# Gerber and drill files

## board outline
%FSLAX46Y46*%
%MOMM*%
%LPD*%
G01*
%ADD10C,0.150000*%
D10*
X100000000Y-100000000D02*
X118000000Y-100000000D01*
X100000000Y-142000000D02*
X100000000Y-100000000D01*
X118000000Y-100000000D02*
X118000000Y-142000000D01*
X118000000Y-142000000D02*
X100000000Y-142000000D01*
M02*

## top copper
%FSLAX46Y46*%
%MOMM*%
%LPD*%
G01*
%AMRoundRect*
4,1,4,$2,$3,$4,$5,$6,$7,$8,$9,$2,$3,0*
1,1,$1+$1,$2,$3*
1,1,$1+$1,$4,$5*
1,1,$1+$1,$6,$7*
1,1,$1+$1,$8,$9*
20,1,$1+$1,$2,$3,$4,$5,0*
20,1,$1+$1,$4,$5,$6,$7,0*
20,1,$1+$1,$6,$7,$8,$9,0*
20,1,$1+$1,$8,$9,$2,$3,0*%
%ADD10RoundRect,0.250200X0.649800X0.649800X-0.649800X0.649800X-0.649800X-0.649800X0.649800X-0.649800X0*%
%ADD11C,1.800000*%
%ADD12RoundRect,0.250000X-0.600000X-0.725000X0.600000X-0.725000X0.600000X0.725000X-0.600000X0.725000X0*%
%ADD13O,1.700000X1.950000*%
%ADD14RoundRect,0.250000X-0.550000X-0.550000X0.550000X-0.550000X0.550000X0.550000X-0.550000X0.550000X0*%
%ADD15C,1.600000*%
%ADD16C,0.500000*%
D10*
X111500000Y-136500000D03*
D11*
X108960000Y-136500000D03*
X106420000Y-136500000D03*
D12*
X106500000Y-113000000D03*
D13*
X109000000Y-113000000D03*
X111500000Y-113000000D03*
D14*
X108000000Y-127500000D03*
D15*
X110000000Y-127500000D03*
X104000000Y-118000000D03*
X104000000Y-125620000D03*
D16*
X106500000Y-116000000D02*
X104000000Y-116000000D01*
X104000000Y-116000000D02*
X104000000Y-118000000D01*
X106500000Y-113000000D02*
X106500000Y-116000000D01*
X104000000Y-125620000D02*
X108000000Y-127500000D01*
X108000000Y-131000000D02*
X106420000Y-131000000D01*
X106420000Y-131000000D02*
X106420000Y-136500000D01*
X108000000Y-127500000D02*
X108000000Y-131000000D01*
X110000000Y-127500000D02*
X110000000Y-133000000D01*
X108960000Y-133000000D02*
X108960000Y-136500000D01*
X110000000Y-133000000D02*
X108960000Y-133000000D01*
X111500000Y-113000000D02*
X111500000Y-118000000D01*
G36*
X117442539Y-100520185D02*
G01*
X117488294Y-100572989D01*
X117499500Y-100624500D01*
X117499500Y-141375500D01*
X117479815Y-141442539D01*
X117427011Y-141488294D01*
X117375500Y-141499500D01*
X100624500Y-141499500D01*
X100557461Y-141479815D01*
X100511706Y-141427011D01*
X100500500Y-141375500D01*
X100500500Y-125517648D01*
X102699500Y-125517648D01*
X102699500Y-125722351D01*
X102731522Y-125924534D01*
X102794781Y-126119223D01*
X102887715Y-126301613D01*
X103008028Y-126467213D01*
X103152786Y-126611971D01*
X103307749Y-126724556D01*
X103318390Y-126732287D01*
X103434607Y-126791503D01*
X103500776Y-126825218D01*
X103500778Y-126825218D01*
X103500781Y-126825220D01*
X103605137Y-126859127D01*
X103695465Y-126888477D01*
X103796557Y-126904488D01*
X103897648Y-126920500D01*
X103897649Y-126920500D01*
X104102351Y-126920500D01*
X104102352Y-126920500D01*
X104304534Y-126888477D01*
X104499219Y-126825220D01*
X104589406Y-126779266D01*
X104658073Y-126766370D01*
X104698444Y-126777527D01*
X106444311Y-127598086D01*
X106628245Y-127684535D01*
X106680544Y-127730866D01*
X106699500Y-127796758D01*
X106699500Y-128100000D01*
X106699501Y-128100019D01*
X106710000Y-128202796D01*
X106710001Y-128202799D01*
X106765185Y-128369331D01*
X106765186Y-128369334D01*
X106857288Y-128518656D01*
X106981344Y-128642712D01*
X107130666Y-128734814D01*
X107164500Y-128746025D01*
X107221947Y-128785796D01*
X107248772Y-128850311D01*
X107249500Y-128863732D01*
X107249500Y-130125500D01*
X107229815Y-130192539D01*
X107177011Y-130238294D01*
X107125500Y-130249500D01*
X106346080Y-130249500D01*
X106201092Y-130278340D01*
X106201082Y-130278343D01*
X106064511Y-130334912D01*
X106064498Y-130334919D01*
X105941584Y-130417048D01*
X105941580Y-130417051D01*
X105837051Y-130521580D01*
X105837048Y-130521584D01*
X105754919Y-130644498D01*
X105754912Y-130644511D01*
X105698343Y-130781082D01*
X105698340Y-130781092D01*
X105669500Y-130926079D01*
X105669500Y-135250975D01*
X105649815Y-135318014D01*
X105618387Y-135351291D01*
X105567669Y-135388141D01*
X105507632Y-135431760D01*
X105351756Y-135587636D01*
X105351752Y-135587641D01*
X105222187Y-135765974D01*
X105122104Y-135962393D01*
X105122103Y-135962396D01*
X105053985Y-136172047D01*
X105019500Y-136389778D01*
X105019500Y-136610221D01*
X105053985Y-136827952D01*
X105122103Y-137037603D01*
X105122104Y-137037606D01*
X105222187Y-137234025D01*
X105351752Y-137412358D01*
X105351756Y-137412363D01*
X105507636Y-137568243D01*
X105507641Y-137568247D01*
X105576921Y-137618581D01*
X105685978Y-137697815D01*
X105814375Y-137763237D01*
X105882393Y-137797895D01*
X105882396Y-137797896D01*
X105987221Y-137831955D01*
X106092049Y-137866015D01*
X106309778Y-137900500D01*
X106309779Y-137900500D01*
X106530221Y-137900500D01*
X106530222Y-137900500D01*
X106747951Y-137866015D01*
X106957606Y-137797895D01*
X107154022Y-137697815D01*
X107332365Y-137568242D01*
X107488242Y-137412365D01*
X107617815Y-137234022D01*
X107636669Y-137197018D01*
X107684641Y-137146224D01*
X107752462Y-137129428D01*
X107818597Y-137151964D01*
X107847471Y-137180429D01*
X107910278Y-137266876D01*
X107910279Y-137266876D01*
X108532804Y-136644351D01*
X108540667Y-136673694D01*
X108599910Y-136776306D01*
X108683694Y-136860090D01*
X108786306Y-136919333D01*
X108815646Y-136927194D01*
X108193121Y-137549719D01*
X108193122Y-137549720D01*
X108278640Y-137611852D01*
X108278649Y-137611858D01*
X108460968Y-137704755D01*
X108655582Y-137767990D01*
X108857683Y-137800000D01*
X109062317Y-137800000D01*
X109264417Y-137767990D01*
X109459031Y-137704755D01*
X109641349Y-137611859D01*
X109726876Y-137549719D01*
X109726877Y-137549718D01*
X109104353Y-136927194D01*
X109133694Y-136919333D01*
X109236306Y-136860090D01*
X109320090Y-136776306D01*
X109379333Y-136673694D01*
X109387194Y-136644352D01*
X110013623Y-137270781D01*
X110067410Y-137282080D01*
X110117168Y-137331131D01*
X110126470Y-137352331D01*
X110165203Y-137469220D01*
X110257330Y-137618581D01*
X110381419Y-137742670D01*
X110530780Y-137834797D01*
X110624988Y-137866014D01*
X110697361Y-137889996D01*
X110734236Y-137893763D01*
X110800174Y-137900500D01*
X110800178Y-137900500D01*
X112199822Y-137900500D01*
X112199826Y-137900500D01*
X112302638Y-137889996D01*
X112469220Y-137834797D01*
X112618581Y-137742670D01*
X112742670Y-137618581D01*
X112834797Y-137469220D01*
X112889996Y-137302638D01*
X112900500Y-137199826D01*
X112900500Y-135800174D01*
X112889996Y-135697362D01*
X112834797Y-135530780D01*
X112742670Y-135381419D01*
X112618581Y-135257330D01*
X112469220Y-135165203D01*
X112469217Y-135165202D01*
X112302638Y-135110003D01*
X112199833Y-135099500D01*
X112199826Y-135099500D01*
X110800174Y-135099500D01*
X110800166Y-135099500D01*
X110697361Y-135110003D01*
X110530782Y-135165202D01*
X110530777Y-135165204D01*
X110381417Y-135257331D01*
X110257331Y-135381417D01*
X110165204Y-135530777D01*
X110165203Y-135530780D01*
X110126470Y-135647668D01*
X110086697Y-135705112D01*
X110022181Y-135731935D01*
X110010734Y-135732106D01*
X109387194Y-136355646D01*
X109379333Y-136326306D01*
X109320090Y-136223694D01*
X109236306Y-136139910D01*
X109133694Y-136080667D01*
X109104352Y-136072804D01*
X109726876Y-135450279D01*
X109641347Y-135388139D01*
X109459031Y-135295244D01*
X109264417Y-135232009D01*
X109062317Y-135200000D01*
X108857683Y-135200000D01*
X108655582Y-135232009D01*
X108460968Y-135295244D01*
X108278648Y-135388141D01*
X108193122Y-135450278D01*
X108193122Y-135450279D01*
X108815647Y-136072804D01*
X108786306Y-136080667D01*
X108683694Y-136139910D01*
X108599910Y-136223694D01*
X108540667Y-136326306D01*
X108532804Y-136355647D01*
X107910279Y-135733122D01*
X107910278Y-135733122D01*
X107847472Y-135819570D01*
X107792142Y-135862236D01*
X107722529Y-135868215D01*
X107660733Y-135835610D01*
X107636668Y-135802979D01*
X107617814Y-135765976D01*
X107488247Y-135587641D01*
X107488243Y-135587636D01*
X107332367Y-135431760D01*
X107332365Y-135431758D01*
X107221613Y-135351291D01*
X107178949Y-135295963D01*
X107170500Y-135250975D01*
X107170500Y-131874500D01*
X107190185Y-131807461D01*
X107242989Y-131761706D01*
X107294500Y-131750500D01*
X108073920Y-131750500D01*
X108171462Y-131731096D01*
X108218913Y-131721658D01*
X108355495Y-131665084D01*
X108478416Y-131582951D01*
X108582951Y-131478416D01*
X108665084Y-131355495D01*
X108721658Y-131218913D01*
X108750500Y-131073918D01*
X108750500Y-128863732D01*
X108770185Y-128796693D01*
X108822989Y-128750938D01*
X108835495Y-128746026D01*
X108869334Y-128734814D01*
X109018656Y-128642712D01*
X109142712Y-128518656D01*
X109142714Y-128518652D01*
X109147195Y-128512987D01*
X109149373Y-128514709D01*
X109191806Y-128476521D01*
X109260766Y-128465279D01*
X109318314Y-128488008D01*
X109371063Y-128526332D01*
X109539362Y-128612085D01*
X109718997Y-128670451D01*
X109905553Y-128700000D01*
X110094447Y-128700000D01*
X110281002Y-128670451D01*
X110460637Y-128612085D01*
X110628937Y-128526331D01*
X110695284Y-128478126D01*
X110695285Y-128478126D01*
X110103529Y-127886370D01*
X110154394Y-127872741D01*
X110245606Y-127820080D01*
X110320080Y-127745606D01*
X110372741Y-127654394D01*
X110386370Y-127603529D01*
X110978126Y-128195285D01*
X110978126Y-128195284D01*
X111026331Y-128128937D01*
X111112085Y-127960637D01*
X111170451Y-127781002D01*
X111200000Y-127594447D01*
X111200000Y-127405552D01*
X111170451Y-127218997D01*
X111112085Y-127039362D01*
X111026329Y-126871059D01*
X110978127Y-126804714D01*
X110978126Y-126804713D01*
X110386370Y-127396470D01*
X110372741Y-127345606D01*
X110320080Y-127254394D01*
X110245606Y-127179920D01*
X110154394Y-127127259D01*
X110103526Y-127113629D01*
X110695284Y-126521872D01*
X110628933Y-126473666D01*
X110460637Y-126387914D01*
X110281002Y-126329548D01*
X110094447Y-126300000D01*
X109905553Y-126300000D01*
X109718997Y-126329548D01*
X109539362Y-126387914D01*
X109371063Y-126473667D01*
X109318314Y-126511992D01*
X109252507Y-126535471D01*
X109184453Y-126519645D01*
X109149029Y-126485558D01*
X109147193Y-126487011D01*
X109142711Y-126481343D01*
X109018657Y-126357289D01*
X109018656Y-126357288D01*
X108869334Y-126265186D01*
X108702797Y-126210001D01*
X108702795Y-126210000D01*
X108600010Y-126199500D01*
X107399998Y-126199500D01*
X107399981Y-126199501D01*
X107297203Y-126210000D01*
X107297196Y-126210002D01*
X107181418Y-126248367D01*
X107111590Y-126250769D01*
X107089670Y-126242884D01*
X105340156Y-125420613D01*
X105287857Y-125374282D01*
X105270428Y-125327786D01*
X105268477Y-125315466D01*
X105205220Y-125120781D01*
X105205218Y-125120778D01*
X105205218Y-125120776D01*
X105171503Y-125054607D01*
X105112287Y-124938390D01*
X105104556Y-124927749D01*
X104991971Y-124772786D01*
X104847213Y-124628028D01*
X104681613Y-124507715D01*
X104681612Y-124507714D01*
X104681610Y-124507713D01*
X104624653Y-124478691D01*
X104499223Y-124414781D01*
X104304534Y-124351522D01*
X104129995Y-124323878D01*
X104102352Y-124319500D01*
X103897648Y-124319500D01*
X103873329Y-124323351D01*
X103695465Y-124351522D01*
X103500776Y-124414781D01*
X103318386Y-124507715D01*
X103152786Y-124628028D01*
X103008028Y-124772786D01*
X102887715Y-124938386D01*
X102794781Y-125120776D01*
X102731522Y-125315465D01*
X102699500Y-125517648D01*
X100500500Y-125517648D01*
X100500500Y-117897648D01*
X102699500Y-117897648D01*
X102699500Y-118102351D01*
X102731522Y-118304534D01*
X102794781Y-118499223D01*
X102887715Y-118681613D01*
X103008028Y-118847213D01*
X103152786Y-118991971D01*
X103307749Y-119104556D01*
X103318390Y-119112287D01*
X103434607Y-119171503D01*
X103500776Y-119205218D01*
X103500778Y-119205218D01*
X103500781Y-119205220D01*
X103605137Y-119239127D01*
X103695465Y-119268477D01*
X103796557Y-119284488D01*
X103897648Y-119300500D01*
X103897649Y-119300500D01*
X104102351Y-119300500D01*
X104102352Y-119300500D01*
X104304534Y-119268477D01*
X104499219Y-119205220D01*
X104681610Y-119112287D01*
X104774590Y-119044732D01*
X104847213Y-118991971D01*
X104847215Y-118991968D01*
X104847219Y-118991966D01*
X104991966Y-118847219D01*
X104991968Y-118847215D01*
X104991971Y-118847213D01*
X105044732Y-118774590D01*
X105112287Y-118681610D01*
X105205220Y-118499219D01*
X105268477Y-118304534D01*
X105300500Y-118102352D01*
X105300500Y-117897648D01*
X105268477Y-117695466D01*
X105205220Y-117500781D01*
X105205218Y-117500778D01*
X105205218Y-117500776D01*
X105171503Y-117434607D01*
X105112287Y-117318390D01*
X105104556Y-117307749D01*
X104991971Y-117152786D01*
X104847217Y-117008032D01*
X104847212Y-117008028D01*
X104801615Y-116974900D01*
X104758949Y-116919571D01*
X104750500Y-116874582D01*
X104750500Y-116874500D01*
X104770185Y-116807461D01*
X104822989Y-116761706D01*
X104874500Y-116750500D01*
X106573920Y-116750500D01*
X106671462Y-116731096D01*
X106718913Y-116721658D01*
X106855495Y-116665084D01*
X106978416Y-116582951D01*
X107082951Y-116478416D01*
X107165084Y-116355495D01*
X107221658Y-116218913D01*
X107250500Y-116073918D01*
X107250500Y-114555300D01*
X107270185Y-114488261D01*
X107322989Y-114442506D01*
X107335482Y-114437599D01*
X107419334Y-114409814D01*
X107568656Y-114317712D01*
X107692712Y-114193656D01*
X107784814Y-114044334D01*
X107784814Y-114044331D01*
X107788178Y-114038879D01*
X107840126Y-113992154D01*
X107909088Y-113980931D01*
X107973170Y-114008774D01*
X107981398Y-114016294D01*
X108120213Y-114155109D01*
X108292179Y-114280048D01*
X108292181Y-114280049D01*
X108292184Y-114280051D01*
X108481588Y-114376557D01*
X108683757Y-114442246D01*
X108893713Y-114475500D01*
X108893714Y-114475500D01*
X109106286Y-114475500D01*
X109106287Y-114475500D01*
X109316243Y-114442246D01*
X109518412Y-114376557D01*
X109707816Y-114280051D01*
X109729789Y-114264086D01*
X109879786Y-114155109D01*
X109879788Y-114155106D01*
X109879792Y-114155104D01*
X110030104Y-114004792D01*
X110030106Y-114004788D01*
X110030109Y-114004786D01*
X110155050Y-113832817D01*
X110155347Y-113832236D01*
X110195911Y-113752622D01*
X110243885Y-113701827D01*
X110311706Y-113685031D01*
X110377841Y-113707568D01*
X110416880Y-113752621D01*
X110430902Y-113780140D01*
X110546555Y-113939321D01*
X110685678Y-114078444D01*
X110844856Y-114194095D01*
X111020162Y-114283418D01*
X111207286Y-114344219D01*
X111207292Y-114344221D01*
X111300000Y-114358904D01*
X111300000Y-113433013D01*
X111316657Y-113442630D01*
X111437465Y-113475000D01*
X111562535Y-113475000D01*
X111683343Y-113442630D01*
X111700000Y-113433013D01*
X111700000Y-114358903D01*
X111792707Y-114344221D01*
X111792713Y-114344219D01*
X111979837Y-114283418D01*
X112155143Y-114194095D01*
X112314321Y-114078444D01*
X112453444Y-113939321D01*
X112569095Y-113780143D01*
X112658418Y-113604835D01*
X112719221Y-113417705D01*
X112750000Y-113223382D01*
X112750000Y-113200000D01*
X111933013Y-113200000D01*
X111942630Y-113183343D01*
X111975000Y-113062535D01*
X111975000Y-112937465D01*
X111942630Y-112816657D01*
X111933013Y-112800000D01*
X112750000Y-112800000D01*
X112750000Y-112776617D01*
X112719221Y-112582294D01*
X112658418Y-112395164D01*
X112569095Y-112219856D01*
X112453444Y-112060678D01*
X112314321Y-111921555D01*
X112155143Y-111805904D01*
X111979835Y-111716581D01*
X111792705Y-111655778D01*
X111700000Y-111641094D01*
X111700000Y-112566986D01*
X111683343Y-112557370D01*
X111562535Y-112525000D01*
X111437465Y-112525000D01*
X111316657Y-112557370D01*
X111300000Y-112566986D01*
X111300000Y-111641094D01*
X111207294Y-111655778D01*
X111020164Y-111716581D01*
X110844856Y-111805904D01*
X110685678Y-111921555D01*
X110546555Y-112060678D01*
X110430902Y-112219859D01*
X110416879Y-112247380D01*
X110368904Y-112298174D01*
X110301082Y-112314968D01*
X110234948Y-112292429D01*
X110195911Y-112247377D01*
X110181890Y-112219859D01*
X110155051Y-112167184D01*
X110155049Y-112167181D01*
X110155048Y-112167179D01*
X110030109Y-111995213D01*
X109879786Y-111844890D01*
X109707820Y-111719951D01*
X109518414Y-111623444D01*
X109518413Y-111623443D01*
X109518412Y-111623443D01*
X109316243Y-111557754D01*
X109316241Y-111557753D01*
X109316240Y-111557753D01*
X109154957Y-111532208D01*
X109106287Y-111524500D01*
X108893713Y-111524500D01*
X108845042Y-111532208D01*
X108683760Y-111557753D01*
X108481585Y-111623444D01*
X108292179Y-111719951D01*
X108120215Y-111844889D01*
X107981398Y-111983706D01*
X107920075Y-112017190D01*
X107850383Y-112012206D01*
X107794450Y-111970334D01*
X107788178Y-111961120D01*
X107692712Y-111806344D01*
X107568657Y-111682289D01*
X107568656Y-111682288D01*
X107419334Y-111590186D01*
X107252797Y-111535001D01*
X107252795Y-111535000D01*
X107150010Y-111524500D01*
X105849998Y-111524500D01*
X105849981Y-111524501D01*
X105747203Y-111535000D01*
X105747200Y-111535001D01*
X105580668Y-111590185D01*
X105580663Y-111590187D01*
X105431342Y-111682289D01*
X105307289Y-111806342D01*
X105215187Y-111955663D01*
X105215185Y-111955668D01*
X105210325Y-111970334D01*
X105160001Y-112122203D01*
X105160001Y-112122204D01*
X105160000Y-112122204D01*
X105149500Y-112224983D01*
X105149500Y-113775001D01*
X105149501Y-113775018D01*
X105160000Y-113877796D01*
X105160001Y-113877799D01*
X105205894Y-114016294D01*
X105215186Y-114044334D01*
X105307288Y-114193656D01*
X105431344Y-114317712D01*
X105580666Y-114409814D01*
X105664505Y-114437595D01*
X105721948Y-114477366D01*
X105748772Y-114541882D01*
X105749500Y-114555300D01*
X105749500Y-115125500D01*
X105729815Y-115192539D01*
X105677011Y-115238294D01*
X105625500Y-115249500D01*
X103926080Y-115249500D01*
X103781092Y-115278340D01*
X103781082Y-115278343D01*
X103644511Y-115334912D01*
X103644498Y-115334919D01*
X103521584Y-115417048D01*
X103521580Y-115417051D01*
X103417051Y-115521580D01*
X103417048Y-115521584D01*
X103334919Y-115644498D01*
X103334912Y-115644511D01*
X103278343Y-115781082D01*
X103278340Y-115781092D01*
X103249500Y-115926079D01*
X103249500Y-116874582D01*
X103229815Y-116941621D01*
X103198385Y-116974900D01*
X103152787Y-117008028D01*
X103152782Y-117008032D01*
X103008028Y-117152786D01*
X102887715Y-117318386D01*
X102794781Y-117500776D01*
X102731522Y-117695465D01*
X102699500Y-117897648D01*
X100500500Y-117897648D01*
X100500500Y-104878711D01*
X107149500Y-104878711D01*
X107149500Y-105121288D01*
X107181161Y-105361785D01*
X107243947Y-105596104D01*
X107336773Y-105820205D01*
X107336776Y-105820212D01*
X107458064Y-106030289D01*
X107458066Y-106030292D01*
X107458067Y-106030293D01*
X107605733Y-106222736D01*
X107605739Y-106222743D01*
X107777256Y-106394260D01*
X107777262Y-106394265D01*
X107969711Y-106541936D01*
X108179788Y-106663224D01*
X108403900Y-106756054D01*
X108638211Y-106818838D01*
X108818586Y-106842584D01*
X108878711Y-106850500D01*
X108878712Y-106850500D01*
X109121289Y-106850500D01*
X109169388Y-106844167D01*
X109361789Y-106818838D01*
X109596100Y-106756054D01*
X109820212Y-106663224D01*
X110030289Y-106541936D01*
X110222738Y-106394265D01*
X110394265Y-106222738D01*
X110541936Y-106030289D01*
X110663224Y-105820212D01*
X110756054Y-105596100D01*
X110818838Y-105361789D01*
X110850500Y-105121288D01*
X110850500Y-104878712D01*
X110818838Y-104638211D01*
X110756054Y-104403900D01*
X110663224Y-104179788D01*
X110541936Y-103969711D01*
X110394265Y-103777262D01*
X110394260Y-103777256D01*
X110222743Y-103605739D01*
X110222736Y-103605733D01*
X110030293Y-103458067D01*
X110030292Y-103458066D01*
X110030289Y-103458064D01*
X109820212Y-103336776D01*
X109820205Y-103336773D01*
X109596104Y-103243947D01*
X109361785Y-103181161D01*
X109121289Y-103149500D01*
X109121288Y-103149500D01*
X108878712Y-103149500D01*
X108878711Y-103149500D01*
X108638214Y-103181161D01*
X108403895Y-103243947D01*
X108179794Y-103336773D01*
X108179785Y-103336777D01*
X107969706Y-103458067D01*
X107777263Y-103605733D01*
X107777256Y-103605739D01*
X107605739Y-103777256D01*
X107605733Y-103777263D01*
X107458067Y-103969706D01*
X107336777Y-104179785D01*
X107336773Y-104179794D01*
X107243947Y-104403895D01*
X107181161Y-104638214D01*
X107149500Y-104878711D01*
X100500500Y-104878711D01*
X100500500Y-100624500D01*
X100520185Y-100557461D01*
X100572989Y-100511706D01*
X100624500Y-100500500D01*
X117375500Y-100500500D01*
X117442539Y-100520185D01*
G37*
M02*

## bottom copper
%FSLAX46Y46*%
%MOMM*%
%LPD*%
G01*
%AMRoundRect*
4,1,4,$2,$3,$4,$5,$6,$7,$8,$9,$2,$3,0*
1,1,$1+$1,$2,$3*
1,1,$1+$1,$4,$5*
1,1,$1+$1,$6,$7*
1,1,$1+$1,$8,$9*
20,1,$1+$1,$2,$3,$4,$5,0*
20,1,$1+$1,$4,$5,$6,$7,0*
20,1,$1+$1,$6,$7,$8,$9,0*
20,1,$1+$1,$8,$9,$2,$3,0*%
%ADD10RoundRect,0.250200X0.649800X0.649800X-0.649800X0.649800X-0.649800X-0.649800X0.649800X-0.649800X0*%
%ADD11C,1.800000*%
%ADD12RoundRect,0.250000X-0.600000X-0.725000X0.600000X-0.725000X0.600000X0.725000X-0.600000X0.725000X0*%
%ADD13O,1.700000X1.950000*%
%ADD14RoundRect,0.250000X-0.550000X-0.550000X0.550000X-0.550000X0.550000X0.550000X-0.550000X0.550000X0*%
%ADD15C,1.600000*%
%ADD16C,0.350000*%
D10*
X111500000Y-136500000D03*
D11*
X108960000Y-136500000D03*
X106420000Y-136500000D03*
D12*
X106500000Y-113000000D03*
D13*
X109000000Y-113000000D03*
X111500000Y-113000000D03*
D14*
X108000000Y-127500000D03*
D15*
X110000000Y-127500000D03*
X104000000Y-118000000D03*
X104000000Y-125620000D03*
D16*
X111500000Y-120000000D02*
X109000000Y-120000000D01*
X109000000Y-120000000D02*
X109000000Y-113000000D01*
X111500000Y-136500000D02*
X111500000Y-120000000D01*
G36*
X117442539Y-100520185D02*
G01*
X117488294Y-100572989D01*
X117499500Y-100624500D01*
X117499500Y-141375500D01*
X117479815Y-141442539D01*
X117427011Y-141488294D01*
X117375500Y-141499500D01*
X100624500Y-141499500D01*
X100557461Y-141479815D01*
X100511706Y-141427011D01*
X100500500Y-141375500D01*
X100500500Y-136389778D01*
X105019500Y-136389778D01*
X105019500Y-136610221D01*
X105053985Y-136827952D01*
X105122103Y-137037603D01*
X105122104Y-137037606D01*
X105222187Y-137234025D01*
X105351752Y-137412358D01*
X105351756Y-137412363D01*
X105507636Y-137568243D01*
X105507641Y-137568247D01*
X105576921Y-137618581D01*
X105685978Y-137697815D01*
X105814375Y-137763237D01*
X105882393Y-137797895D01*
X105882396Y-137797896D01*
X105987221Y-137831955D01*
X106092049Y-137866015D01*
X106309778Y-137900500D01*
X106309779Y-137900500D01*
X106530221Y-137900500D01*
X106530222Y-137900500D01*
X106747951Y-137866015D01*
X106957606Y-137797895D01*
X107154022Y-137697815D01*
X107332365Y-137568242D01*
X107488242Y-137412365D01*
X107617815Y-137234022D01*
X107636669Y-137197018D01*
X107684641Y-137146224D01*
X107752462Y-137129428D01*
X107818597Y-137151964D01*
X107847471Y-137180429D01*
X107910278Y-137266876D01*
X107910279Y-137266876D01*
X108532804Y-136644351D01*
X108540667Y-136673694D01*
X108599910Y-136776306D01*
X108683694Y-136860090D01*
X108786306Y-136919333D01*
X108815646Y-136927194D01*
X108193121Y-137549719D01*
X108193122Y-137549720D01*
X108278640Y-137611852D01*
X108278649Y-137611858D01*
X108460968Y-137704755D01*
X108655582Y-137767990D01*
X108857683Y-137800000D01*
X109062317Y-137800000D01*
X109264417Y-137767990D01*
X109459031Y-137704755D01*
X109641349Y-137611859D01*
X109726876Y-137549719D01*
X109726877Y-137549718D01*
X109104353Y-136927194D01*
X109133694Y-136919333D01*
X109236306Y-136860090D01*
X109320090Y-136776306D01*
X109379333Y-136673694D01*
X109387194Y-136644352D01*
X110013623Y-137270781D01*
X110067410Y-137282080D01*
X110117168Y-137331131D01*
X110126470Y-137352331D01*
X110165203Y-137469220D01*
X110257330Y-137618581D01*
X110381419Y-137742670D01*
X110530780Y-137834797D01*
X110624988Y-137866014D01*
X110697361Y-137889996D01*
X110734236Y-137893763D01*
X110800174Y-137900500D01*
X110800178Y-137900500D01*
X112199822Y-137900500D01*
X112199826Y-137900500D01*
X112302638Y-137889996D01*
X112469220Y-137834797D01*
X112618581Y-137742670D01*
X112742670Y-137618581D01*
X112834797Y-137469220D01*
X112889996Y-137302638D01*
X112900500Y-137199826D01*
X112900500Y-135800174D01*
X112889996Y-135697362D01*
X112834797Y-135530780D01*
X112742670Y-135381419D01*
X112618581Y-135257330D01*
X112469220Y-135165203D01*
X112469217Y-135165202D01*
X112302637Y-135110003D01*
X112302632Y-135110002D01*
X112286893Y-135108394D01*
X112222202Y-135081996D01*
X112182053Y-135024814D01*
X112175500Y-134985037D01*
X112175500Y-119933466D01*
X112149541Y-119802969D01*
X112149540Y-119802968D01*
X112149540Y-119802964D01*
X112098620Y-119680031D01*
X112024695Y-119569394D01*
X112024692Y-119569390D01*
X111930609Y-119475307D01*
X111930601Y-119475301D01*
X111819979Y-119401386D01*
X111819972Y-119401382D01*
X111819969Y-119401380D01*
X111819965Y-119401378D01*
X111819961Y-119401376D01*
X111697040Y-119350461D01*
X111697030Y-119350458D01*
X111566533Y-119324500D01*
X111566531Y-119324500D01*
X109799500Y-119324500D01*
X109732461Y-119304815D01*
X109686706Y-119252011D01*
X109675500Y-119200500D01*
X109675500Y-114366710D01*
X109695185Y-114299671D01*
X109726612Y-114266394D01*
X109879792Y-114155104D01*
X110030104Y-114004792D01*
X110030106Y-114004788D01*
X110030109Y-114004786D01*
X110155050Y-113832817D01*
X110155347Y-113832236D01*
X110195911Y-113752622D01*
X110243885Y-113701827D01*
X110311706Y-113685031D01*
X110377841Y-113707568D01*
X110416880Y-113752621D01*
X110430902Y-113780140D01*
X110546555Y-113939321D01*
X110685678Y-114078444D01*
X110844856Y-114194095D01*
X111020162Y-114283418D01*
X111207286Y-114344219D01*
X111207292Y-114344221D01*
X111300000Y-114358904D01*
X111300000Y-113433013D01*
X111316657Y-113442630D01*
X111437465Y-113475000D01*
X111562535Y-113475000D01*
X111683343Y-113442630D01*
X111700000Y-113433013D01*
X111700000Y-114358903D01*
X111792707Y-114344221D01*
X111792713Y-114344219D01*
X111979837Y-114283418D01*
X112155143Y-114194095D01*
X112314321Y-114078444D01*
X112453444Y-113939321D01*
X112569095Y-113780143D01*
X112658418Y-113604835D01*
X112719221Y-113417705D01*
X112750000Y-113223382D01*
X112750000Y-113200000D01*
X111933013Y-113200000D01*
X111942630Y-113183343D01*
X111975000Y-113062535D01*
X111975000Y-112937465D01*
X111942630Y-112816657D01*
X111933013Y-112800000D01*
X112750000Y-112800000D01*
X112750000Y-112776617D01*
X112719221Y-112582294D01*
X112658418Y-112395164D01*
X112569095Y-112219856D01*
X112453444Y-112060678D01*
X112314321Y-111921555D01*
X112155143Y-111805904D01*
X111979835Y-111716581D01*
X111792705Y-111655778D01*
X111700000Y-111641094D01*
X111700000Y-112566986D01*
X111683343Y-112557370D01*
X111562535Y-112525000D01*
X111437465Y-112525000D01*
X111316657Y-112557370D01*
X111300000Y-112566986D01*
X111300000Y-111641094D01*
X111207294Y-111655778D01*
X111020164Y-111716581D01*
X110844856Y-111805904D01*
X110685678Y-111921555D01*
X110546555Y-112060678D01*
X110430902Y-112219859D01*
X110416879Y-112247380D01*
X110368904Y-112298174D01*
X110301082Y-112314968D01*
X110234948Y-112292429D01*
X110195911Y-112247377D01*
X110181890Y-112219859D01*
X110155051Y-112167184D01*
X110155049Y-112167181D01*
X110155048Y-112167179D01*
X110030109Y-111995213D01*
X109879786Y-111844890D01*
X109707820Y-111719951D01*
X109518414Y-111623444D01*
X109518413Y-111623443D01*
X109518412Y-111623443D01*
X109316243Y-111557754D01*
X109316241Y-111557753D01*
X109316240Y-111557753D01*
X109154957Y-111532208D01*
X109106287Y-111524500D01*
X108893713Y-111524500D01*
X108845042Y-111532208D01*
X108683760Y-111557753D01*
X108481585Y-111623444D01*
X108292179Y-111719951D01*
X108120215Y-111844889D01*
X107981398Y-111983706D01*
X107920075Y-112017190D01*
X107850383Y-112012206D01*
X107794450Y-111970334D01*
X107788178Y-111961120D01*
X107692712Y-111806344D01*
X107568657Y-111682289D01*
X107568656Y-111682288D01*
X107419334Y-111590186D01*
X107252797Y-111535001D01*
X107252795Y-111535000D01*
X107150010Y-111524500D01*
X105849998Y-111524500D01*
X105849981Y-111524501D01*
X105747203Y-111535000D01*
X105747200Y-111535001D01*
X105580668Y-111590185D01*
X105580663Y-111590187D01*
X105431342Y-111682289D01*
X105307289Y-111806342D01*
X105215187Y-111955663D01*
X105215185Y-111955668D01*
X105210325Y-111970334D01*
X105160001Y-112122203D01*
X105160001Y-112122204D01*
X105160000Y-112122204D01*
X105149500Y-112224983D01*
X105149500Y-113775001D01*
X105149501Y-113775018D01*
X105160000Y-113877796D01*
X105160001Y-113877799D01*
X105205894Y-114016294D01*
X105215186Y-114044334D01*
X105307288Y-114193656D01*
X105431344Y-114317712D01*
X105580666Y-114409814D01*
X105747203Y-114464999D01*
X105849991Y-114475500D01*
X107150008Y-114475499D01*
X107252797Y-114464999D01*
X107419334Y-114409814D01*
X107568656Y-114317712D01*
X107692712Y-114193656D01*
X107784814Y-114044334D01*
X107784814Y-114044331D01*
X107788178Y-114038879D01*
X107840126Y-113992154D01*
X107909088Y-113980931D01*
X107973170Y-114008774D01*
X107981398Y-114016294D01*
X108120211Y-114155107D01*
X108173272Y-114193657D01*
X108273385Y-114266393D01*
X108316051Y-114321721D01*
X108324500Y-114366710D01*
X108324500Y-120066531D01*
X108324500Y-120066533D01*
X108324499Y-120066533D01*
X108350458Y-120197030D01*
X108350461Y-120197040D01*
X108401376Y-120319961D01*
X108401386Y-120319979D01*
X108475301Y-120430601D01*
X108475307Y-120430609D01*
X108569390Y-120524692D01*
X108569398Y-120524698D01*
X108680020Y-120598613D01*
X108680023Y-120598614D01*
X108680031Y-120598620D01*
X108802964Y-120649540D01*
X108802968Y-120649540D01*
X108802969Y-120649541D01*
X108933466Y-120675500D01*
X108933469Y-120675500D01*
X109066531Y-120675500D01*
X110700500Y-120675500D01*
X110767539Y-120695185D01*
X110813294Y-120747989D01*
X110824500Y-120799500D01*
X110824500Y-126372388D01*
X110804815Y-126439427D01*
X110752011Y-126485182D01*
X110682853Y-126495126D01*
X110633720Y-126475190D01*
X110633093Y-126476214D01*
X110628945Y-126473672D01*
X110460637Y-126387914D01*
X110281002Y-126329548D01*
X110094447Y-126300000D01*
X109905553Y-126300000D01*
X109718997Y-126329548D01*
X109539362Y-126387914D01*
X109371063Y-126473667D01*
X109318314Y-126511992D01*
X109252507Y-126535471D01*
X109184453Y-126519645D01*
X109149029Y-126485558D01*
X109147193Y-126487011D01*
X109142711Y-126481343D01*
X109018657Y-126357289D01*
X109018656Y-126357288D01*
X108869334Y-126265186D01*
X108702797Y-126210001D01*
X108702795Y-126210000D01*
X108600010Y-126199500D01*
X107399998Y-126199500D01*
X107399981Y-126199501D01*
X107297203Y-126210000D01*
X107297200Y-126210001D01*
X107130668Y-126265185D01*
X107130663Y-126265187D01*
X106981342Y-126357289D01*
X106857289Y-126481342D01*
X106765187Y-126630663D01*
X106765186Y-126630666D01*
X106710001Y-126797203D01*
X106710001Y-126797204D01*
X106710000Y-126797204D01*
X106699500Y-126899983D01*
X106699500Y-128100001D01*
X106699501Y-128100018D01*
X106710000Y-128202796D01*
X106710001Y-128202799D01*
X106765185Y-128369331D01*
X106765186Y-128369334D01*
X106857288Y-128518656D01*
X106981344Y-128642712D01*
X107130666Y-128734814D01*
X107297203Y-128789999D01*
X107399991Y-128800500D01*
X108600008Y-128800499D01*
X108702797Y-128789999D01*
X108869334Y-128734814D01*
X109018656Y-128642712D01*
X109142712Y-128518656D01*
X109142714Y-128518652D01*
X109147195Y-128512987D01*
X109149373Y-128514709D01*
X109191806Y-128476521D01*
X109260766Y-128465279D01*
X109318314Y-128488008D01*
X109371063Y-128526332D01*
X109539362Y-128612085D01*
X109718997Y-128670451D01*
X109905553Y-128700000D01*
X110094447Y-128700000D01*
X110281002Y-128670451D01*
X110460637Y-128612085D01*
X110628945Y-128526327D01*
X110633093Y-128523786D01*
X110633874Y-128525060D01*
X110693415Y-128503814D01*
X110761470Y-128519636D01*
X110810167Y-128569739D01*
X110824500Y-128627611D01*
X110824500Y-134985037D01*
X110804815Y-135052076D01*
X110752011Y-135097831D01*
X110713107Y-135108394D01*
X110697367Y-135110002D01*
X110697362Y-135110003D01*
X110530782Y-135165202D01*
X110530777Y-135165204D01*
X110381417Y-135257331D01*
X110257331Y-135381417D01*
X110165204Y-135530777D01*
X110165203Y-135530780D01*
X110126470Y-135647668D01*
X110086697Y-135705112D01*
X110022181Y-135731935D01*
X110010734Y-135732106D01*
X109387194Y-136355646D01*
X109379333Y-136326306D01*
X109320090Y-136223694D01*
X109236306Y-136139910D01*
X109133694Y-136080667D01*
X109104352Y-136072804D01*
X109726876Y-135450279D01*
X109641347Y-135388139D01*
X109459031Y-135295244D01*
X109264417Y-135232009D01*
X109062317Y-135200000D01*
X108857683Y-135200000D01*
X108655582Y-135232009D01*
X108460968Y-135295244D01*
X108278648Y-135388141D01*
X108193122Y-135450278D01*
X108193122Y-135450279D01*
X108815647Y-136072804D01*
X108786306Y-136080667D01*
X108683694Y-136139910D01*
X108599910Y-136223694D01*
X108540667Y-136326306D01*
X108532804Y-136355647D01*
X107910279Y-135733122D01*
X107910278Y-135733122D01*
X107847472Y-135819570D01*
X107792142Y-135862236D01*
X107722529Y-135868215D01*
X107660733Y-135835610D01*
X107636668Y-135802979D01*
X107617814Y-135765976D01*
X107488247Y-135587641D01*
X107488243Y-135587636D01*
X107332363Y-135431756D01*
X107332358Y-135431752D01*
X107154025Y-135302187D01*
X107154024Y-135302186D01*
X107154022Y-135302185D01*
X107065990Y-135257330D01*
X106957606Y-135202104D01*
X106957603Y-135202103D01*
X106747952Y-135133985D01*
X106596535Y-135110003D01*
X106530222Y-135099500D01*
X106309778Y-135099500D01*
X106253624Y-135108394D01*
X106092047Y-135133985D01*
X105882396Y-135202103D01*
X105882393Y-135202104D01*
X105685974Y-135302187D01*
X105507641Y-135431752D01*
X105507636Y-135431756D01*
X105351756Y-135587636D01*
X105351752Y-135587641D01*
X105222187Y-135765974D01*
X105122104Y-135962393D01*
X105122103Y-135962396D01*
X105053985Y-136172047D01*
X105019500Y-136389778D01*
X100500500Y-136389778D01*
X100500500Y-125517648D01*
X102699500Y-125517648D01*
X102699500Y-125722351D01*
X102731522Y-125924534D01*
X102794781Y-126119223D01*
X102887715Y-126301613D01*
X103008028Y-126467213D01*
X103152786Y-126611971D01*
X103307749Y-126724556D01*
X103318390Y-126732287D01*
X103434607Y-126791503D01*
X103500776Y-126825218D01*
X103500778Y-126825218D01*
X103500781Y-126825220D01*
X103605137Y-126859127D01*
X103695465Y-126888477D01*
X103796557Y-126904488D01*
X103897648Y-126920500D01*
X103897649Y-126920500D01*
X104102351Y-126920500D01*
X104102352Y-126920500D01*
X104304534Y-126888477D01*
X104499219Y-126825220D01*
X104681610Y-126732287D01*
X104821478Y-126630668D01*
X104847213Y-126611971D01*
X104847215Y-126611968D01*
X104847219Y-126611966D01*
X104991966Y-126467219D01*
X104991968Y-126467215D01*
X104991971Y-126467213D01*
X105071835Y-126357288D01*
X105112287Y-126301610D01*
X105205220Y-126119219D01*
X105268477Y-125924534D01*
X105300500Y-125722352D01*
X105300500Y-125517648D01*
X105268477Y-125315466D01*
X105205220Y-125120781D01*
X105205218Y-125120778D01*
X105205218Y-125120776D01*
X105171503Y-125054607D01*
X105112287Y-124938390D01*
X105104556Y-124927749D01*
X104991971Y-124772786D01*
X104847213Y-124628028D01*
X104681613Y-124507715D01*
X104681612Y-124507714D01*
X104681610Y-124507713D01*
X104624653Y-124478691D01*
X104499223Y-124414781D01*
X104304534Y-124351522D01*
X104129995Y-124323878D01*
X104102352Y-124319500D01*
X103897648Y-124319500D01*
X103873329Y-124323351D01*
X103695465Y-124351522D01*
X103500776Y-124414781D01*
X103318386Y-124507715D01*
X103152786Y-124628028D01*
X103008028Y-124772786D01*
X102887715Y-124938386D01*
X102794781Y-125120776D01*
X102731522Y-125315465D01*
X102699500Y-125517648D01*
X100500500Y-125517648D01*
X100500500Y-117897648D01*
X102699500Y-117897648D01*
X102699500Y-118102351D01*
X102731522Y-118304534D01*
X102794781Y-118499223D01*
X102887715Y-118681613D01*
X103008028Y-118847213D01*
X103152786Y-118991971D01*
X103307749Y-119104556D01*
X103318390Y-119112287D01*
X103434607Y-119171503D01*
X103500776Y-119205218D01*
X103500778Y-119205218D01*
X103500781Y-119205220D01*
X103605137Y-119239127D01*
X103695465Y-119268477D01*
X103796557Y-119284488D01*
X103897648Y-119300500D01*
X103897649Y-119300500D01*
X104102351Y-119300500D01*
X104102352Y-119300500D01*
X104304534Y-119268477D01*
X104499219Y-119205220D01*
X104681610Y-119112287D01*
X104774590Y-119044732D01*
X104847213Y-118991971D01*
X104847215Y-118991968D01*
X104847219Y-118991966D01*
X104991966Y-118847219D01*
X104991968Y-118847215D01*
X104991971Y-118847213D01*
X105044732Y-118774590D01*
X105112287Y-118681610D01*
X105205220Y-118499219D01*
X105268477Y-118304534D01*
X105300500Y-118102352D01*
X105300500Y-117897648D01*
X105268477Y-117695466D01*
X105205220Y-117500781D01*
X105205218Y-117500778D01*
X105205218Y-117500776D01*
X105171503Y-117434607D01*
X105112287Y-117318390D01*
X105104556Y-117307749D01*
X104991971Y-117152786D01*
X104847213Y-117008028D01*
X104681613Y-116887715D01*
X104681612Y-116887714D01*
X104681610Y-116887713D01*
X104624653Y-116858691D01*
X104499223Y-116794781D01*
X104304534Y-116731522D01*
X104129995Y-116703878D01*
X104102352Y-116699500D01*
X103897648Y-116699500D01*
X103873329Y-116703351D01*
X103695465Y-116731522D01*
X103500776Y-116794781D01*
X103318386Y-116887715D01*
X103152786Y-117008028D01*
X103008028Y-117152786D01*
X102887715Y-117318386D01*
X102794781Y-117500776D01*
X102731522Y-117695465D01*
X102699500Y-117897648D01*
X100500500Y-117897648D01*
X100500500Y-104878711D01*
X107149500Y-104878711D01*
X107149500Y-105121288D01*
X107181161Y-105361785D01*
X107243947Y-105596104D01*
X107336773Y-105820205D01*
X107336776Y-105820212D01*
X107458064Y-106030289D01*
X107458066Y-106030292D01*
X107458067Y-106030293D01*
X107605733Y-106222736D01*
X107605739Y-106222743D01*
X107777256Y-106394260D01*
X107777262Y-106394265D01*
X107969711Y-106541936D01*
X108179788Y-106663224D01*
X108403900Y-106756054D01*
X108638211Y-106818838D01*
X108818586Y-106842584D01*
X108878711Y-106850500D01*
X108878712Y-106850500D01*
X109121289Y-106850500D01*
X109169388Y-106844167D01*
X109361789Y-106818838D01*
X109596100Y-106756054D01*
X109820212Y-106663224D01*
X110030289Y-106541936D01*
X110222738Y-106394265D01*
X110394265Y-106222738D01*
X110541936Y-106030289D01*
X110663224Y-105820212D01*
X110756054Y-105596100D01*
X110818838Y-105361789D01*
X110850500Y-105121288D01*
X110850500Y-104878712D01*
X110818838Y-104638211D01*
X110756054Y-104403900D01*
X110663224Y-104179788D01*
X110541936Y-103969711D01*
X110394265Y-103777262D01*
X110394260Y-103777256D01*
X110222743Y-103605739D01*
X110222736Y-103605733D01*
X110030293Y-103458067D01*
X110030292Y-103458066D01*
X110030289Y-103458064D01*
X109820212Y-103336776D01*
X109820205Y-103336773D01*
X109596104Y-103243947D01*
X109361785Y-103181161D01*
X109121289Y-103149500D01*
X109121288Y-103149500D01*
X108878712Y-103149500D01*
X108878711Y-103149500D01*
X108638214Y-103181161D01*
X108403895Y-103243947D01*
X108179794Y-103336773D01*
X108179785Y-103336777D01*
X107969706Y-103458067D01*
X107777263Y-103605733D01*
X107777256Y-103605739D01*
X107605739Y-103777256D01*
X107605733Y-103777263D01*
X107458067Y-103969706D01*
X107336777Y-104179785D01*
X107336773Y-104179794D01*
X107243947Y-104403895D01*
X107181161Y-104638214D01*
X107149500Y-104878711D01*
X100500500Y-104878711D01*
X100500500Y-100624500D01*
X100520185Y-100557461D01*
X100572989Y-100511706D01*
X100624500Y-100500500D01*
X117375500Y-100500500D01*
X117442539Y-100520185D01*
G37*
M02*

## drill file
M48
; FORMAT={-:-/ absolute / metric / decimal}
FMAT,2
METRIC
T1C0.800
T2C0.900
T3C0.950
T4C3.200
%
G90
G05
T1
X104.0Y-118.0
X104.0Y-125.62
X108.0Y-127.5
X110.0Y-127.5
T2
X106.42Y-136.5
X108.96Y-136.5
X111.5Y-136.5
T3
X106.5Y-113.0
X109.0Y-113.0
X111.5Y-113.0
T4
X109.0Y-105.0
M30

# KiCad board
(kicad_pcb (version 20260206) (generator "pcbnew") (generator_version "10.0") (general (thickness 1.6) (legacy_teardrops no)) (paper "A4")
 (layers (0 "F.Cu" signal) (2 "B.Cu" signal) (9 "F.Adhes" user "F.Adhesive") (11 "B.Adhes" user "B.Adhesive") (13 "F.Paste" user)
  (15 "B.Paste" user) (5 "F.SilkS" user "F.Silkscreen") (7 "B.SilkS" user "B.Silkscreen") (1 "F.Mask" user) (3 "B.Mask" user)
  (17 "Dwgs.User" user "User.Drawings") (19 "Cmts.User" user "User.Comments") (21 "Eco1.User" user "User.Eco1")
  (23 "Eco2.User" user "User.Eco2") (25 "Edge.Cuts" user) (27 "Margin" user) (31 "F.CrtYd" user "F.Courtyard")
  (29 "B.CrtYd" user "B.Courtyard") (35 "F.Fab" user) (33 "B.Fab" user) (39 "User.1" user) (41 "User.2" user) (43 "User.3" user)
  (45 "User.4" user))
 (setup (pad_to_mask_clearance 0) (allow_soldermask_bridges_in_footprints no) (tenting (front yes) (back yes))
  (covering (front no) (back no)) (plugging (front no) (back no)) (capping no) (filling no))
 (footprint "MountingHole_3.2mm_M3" (layer "F.Cu") (at 109 105)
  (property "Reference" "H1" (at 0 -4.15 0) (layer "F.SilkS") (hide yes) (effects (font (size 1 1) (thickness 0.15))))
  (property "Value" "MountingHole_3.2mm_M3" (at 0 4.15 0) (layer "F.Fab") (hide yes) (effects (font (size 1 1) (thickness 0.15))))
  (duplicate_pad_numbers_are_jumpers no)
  (pad "" np_thru_hole circle (at 0 0) (size 3.2 3.2) (drill 3.2) (layers "*.Cu" "*.Mask")))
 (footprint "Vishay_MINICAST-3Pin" (layer "F.Cu") (at 111.5 136.5 180)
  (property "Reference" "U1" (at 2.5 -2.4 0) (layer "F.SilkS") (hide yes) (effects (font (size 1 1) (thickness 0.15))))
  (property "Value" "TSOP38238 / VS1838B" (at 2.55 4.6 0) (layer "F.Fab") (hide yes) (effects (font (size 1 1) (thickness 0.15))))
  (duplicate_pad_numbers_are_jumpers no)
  (pad "1" thru_hole roundrect (at 0 0 180) (size 1.8 1.8) (drill 0.9) (layers "*.Cu" "*.Mask") (remove_unused_layers no)
   (roundrect_rratio 0.139) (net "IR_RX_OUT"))
  (pad "2" thru_hole circle (at 2.54 0 180) (size 1.8 1.8) (drill 0.9) (layers "*.Cu" "*.Mask") (remove_unused_layers no) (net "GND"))
  (pad "3" thru_hole circle (at 5.08 0 180) (size 1.8 1.8) (drill 0.9) (layers "*.Cu" "*.Mask") (remove_unused_layers no) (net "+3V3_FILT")))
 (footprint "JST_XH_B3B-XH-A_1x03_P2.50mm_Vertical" (layer "F.Cu") (at 106.5 113)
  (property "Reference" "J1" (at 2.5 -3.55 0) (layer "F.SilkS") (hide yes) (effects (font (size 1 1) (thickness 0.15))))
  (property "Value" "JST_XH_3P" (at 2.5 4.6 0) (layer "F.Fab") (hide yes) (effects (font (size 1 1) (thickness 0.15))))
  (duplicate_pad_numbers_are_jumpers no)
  (pad "1" thru_hole roundrect (at 0 0) (size 1.7 1.95) (drill 0.95) (layers "*.Cu" "*.Mask") (remove_unused_layers no)
   (roundrect_rratio 0.147059) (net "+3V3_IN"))
  (pad "2" thru_hole oval (at 2.5 0) (size 1.7 1.95) (drill 0.95) (layers "*.Cu" "*.Mask") (remove_unused_layers no) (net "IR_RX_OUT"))
  (pad "3" thru_hole oval (at 5 0) (size 1.7 1.95) (drill 0.95) (layers "*.Cu" "*.Mask") (remove_unused_layers no) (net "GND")))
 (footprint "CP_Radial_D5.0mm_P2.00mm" (layer "F.Cu") (at 108 127.5)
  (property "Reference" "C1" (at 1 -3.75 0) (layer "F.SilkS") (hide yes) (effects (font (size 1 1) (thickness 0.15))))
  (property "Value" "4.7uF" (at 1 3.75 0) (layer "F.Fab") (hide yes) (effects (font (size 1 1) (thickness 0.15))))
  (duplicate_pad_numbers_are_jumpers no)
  (pad "1" thru_hole roundrect (at 0 0) (size 1.6 1.6) (drill 0.8) (layers "*.Cu" "*.Mask") (remove_unused_layers no)
   (roundrect_rratio 0.15625) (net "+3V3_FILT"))
  (pad "2" thru_hole circle (at 2 0) (size 1.6 1.6) (drill 0.8) (layers "*.Cu" "*.Mask") (remove_unused_layers no) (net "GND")))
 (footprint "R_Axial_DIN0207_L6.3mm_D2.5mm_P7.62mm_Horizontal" (layer "F.Cu") (at 104 118 -90)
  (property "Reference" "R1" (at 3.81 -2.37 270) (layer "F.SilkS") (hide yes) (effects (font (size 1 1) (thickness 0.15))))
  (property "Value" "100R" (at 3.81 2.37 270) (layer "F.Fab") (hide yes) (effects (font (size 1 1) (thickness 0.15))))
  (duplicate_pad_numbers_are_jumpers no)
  (pad "1" thru_hole circle (at 0 0 270) (size 1.6 1.6) (drill 0.8) (layers "*.Cu" "*.Mask") (remove_unused_layers no) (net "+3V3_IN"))
  (pad "2" thru_hole circle (at 7.62 0 270) (size 1.6 1.6) (drill 0.8) (layers "*.Cu" "*.Mask") (remove_unused_layers no) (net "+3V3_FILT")))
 (gr_line (start 100 100) (end 118 100) (stroke (width 0.15) (type default)) (layer "Edge.Cuts"))
 (gr_line (start 100 142) (end 100 100) (stroke (width 0.15) (type default)) (layer "Edge.Cuts"))
 (gr_line (start 118 100) (end 118 142) (stroke (width 0.15) (type default)) (layer "Edge.Cuts"))
 (gr_line (start 118 142) (end 100 142) (stroke (width 0.15) (type default)) (layer "Edge.Cuts"))
 (segment (start 106.5 116) (end 104 116) (width 0.5) (layer "F.Cu") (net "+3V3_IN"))
 (segment (start 104 116) (end 104 118) (width 0.5) (layer "F.Cu") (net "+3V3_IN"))
 (segment (start 106.5 113) (end 106.5 116) (width 0.5) (layer "F.Cu") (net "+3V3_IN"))
 (segment (start 104 125.62) (end 108 127.5) (width 0.5) (layer "F.Cu") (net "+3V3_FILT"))
 (segment (start 108 131) (end 106.42 131) (width 0.5) (layer "F.Cu") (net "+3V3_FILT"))
 (segment (start 106.42 131) (end 106.42 136.5) (width 0.5) (layer "F.Cu") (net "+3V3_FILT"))
 (segment (start 108 127.5) (end 108 131) (width 0.5) (layer "F.Cu") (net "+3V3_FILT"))
 (segment (start 111.5 120) (end 109 120) (width 0.35) (layer "B.Cu") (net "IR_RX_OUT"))
 (segment (start 109 120) (end 109 113) (width 0.35) (layer "B.Cu") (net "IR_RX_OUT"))
 (segment (start 111.5 136.5) (end 111.5 120) (width 0.35) (layer "B.Cu") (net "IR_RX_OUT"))
 (segment (start 110 127.5) (end 110 133) (width 0.5) (layer "F.Cu") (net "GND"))
 (segment (start 108.96 133) (end 108.96 136.5) (width 0.5) (layer "F.Cu") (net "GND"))
 (segment (start 110 133) (end 108.96 133) (width 0.5) (layer "F.Cu") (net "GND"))
 (segment (start 111.5 113) (end 111.5 118) (width 0.5) (layer "F.Cu") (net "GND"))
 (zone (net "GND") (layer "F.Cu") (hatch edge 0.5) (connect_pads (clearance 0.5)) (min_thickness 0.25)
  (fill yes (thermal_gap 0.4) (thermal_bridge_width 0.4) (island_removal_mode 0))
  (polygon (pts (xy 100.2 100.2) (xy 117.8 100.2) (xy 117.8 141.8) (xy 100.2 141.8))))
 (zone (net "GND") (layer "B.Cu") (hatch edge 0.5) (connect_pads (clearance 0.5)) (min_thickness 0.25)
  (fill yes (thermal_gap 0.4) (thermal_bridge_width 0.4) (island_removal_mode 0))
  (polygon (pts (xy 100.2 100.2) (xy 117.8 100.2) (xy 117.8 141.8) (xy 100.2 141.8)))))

